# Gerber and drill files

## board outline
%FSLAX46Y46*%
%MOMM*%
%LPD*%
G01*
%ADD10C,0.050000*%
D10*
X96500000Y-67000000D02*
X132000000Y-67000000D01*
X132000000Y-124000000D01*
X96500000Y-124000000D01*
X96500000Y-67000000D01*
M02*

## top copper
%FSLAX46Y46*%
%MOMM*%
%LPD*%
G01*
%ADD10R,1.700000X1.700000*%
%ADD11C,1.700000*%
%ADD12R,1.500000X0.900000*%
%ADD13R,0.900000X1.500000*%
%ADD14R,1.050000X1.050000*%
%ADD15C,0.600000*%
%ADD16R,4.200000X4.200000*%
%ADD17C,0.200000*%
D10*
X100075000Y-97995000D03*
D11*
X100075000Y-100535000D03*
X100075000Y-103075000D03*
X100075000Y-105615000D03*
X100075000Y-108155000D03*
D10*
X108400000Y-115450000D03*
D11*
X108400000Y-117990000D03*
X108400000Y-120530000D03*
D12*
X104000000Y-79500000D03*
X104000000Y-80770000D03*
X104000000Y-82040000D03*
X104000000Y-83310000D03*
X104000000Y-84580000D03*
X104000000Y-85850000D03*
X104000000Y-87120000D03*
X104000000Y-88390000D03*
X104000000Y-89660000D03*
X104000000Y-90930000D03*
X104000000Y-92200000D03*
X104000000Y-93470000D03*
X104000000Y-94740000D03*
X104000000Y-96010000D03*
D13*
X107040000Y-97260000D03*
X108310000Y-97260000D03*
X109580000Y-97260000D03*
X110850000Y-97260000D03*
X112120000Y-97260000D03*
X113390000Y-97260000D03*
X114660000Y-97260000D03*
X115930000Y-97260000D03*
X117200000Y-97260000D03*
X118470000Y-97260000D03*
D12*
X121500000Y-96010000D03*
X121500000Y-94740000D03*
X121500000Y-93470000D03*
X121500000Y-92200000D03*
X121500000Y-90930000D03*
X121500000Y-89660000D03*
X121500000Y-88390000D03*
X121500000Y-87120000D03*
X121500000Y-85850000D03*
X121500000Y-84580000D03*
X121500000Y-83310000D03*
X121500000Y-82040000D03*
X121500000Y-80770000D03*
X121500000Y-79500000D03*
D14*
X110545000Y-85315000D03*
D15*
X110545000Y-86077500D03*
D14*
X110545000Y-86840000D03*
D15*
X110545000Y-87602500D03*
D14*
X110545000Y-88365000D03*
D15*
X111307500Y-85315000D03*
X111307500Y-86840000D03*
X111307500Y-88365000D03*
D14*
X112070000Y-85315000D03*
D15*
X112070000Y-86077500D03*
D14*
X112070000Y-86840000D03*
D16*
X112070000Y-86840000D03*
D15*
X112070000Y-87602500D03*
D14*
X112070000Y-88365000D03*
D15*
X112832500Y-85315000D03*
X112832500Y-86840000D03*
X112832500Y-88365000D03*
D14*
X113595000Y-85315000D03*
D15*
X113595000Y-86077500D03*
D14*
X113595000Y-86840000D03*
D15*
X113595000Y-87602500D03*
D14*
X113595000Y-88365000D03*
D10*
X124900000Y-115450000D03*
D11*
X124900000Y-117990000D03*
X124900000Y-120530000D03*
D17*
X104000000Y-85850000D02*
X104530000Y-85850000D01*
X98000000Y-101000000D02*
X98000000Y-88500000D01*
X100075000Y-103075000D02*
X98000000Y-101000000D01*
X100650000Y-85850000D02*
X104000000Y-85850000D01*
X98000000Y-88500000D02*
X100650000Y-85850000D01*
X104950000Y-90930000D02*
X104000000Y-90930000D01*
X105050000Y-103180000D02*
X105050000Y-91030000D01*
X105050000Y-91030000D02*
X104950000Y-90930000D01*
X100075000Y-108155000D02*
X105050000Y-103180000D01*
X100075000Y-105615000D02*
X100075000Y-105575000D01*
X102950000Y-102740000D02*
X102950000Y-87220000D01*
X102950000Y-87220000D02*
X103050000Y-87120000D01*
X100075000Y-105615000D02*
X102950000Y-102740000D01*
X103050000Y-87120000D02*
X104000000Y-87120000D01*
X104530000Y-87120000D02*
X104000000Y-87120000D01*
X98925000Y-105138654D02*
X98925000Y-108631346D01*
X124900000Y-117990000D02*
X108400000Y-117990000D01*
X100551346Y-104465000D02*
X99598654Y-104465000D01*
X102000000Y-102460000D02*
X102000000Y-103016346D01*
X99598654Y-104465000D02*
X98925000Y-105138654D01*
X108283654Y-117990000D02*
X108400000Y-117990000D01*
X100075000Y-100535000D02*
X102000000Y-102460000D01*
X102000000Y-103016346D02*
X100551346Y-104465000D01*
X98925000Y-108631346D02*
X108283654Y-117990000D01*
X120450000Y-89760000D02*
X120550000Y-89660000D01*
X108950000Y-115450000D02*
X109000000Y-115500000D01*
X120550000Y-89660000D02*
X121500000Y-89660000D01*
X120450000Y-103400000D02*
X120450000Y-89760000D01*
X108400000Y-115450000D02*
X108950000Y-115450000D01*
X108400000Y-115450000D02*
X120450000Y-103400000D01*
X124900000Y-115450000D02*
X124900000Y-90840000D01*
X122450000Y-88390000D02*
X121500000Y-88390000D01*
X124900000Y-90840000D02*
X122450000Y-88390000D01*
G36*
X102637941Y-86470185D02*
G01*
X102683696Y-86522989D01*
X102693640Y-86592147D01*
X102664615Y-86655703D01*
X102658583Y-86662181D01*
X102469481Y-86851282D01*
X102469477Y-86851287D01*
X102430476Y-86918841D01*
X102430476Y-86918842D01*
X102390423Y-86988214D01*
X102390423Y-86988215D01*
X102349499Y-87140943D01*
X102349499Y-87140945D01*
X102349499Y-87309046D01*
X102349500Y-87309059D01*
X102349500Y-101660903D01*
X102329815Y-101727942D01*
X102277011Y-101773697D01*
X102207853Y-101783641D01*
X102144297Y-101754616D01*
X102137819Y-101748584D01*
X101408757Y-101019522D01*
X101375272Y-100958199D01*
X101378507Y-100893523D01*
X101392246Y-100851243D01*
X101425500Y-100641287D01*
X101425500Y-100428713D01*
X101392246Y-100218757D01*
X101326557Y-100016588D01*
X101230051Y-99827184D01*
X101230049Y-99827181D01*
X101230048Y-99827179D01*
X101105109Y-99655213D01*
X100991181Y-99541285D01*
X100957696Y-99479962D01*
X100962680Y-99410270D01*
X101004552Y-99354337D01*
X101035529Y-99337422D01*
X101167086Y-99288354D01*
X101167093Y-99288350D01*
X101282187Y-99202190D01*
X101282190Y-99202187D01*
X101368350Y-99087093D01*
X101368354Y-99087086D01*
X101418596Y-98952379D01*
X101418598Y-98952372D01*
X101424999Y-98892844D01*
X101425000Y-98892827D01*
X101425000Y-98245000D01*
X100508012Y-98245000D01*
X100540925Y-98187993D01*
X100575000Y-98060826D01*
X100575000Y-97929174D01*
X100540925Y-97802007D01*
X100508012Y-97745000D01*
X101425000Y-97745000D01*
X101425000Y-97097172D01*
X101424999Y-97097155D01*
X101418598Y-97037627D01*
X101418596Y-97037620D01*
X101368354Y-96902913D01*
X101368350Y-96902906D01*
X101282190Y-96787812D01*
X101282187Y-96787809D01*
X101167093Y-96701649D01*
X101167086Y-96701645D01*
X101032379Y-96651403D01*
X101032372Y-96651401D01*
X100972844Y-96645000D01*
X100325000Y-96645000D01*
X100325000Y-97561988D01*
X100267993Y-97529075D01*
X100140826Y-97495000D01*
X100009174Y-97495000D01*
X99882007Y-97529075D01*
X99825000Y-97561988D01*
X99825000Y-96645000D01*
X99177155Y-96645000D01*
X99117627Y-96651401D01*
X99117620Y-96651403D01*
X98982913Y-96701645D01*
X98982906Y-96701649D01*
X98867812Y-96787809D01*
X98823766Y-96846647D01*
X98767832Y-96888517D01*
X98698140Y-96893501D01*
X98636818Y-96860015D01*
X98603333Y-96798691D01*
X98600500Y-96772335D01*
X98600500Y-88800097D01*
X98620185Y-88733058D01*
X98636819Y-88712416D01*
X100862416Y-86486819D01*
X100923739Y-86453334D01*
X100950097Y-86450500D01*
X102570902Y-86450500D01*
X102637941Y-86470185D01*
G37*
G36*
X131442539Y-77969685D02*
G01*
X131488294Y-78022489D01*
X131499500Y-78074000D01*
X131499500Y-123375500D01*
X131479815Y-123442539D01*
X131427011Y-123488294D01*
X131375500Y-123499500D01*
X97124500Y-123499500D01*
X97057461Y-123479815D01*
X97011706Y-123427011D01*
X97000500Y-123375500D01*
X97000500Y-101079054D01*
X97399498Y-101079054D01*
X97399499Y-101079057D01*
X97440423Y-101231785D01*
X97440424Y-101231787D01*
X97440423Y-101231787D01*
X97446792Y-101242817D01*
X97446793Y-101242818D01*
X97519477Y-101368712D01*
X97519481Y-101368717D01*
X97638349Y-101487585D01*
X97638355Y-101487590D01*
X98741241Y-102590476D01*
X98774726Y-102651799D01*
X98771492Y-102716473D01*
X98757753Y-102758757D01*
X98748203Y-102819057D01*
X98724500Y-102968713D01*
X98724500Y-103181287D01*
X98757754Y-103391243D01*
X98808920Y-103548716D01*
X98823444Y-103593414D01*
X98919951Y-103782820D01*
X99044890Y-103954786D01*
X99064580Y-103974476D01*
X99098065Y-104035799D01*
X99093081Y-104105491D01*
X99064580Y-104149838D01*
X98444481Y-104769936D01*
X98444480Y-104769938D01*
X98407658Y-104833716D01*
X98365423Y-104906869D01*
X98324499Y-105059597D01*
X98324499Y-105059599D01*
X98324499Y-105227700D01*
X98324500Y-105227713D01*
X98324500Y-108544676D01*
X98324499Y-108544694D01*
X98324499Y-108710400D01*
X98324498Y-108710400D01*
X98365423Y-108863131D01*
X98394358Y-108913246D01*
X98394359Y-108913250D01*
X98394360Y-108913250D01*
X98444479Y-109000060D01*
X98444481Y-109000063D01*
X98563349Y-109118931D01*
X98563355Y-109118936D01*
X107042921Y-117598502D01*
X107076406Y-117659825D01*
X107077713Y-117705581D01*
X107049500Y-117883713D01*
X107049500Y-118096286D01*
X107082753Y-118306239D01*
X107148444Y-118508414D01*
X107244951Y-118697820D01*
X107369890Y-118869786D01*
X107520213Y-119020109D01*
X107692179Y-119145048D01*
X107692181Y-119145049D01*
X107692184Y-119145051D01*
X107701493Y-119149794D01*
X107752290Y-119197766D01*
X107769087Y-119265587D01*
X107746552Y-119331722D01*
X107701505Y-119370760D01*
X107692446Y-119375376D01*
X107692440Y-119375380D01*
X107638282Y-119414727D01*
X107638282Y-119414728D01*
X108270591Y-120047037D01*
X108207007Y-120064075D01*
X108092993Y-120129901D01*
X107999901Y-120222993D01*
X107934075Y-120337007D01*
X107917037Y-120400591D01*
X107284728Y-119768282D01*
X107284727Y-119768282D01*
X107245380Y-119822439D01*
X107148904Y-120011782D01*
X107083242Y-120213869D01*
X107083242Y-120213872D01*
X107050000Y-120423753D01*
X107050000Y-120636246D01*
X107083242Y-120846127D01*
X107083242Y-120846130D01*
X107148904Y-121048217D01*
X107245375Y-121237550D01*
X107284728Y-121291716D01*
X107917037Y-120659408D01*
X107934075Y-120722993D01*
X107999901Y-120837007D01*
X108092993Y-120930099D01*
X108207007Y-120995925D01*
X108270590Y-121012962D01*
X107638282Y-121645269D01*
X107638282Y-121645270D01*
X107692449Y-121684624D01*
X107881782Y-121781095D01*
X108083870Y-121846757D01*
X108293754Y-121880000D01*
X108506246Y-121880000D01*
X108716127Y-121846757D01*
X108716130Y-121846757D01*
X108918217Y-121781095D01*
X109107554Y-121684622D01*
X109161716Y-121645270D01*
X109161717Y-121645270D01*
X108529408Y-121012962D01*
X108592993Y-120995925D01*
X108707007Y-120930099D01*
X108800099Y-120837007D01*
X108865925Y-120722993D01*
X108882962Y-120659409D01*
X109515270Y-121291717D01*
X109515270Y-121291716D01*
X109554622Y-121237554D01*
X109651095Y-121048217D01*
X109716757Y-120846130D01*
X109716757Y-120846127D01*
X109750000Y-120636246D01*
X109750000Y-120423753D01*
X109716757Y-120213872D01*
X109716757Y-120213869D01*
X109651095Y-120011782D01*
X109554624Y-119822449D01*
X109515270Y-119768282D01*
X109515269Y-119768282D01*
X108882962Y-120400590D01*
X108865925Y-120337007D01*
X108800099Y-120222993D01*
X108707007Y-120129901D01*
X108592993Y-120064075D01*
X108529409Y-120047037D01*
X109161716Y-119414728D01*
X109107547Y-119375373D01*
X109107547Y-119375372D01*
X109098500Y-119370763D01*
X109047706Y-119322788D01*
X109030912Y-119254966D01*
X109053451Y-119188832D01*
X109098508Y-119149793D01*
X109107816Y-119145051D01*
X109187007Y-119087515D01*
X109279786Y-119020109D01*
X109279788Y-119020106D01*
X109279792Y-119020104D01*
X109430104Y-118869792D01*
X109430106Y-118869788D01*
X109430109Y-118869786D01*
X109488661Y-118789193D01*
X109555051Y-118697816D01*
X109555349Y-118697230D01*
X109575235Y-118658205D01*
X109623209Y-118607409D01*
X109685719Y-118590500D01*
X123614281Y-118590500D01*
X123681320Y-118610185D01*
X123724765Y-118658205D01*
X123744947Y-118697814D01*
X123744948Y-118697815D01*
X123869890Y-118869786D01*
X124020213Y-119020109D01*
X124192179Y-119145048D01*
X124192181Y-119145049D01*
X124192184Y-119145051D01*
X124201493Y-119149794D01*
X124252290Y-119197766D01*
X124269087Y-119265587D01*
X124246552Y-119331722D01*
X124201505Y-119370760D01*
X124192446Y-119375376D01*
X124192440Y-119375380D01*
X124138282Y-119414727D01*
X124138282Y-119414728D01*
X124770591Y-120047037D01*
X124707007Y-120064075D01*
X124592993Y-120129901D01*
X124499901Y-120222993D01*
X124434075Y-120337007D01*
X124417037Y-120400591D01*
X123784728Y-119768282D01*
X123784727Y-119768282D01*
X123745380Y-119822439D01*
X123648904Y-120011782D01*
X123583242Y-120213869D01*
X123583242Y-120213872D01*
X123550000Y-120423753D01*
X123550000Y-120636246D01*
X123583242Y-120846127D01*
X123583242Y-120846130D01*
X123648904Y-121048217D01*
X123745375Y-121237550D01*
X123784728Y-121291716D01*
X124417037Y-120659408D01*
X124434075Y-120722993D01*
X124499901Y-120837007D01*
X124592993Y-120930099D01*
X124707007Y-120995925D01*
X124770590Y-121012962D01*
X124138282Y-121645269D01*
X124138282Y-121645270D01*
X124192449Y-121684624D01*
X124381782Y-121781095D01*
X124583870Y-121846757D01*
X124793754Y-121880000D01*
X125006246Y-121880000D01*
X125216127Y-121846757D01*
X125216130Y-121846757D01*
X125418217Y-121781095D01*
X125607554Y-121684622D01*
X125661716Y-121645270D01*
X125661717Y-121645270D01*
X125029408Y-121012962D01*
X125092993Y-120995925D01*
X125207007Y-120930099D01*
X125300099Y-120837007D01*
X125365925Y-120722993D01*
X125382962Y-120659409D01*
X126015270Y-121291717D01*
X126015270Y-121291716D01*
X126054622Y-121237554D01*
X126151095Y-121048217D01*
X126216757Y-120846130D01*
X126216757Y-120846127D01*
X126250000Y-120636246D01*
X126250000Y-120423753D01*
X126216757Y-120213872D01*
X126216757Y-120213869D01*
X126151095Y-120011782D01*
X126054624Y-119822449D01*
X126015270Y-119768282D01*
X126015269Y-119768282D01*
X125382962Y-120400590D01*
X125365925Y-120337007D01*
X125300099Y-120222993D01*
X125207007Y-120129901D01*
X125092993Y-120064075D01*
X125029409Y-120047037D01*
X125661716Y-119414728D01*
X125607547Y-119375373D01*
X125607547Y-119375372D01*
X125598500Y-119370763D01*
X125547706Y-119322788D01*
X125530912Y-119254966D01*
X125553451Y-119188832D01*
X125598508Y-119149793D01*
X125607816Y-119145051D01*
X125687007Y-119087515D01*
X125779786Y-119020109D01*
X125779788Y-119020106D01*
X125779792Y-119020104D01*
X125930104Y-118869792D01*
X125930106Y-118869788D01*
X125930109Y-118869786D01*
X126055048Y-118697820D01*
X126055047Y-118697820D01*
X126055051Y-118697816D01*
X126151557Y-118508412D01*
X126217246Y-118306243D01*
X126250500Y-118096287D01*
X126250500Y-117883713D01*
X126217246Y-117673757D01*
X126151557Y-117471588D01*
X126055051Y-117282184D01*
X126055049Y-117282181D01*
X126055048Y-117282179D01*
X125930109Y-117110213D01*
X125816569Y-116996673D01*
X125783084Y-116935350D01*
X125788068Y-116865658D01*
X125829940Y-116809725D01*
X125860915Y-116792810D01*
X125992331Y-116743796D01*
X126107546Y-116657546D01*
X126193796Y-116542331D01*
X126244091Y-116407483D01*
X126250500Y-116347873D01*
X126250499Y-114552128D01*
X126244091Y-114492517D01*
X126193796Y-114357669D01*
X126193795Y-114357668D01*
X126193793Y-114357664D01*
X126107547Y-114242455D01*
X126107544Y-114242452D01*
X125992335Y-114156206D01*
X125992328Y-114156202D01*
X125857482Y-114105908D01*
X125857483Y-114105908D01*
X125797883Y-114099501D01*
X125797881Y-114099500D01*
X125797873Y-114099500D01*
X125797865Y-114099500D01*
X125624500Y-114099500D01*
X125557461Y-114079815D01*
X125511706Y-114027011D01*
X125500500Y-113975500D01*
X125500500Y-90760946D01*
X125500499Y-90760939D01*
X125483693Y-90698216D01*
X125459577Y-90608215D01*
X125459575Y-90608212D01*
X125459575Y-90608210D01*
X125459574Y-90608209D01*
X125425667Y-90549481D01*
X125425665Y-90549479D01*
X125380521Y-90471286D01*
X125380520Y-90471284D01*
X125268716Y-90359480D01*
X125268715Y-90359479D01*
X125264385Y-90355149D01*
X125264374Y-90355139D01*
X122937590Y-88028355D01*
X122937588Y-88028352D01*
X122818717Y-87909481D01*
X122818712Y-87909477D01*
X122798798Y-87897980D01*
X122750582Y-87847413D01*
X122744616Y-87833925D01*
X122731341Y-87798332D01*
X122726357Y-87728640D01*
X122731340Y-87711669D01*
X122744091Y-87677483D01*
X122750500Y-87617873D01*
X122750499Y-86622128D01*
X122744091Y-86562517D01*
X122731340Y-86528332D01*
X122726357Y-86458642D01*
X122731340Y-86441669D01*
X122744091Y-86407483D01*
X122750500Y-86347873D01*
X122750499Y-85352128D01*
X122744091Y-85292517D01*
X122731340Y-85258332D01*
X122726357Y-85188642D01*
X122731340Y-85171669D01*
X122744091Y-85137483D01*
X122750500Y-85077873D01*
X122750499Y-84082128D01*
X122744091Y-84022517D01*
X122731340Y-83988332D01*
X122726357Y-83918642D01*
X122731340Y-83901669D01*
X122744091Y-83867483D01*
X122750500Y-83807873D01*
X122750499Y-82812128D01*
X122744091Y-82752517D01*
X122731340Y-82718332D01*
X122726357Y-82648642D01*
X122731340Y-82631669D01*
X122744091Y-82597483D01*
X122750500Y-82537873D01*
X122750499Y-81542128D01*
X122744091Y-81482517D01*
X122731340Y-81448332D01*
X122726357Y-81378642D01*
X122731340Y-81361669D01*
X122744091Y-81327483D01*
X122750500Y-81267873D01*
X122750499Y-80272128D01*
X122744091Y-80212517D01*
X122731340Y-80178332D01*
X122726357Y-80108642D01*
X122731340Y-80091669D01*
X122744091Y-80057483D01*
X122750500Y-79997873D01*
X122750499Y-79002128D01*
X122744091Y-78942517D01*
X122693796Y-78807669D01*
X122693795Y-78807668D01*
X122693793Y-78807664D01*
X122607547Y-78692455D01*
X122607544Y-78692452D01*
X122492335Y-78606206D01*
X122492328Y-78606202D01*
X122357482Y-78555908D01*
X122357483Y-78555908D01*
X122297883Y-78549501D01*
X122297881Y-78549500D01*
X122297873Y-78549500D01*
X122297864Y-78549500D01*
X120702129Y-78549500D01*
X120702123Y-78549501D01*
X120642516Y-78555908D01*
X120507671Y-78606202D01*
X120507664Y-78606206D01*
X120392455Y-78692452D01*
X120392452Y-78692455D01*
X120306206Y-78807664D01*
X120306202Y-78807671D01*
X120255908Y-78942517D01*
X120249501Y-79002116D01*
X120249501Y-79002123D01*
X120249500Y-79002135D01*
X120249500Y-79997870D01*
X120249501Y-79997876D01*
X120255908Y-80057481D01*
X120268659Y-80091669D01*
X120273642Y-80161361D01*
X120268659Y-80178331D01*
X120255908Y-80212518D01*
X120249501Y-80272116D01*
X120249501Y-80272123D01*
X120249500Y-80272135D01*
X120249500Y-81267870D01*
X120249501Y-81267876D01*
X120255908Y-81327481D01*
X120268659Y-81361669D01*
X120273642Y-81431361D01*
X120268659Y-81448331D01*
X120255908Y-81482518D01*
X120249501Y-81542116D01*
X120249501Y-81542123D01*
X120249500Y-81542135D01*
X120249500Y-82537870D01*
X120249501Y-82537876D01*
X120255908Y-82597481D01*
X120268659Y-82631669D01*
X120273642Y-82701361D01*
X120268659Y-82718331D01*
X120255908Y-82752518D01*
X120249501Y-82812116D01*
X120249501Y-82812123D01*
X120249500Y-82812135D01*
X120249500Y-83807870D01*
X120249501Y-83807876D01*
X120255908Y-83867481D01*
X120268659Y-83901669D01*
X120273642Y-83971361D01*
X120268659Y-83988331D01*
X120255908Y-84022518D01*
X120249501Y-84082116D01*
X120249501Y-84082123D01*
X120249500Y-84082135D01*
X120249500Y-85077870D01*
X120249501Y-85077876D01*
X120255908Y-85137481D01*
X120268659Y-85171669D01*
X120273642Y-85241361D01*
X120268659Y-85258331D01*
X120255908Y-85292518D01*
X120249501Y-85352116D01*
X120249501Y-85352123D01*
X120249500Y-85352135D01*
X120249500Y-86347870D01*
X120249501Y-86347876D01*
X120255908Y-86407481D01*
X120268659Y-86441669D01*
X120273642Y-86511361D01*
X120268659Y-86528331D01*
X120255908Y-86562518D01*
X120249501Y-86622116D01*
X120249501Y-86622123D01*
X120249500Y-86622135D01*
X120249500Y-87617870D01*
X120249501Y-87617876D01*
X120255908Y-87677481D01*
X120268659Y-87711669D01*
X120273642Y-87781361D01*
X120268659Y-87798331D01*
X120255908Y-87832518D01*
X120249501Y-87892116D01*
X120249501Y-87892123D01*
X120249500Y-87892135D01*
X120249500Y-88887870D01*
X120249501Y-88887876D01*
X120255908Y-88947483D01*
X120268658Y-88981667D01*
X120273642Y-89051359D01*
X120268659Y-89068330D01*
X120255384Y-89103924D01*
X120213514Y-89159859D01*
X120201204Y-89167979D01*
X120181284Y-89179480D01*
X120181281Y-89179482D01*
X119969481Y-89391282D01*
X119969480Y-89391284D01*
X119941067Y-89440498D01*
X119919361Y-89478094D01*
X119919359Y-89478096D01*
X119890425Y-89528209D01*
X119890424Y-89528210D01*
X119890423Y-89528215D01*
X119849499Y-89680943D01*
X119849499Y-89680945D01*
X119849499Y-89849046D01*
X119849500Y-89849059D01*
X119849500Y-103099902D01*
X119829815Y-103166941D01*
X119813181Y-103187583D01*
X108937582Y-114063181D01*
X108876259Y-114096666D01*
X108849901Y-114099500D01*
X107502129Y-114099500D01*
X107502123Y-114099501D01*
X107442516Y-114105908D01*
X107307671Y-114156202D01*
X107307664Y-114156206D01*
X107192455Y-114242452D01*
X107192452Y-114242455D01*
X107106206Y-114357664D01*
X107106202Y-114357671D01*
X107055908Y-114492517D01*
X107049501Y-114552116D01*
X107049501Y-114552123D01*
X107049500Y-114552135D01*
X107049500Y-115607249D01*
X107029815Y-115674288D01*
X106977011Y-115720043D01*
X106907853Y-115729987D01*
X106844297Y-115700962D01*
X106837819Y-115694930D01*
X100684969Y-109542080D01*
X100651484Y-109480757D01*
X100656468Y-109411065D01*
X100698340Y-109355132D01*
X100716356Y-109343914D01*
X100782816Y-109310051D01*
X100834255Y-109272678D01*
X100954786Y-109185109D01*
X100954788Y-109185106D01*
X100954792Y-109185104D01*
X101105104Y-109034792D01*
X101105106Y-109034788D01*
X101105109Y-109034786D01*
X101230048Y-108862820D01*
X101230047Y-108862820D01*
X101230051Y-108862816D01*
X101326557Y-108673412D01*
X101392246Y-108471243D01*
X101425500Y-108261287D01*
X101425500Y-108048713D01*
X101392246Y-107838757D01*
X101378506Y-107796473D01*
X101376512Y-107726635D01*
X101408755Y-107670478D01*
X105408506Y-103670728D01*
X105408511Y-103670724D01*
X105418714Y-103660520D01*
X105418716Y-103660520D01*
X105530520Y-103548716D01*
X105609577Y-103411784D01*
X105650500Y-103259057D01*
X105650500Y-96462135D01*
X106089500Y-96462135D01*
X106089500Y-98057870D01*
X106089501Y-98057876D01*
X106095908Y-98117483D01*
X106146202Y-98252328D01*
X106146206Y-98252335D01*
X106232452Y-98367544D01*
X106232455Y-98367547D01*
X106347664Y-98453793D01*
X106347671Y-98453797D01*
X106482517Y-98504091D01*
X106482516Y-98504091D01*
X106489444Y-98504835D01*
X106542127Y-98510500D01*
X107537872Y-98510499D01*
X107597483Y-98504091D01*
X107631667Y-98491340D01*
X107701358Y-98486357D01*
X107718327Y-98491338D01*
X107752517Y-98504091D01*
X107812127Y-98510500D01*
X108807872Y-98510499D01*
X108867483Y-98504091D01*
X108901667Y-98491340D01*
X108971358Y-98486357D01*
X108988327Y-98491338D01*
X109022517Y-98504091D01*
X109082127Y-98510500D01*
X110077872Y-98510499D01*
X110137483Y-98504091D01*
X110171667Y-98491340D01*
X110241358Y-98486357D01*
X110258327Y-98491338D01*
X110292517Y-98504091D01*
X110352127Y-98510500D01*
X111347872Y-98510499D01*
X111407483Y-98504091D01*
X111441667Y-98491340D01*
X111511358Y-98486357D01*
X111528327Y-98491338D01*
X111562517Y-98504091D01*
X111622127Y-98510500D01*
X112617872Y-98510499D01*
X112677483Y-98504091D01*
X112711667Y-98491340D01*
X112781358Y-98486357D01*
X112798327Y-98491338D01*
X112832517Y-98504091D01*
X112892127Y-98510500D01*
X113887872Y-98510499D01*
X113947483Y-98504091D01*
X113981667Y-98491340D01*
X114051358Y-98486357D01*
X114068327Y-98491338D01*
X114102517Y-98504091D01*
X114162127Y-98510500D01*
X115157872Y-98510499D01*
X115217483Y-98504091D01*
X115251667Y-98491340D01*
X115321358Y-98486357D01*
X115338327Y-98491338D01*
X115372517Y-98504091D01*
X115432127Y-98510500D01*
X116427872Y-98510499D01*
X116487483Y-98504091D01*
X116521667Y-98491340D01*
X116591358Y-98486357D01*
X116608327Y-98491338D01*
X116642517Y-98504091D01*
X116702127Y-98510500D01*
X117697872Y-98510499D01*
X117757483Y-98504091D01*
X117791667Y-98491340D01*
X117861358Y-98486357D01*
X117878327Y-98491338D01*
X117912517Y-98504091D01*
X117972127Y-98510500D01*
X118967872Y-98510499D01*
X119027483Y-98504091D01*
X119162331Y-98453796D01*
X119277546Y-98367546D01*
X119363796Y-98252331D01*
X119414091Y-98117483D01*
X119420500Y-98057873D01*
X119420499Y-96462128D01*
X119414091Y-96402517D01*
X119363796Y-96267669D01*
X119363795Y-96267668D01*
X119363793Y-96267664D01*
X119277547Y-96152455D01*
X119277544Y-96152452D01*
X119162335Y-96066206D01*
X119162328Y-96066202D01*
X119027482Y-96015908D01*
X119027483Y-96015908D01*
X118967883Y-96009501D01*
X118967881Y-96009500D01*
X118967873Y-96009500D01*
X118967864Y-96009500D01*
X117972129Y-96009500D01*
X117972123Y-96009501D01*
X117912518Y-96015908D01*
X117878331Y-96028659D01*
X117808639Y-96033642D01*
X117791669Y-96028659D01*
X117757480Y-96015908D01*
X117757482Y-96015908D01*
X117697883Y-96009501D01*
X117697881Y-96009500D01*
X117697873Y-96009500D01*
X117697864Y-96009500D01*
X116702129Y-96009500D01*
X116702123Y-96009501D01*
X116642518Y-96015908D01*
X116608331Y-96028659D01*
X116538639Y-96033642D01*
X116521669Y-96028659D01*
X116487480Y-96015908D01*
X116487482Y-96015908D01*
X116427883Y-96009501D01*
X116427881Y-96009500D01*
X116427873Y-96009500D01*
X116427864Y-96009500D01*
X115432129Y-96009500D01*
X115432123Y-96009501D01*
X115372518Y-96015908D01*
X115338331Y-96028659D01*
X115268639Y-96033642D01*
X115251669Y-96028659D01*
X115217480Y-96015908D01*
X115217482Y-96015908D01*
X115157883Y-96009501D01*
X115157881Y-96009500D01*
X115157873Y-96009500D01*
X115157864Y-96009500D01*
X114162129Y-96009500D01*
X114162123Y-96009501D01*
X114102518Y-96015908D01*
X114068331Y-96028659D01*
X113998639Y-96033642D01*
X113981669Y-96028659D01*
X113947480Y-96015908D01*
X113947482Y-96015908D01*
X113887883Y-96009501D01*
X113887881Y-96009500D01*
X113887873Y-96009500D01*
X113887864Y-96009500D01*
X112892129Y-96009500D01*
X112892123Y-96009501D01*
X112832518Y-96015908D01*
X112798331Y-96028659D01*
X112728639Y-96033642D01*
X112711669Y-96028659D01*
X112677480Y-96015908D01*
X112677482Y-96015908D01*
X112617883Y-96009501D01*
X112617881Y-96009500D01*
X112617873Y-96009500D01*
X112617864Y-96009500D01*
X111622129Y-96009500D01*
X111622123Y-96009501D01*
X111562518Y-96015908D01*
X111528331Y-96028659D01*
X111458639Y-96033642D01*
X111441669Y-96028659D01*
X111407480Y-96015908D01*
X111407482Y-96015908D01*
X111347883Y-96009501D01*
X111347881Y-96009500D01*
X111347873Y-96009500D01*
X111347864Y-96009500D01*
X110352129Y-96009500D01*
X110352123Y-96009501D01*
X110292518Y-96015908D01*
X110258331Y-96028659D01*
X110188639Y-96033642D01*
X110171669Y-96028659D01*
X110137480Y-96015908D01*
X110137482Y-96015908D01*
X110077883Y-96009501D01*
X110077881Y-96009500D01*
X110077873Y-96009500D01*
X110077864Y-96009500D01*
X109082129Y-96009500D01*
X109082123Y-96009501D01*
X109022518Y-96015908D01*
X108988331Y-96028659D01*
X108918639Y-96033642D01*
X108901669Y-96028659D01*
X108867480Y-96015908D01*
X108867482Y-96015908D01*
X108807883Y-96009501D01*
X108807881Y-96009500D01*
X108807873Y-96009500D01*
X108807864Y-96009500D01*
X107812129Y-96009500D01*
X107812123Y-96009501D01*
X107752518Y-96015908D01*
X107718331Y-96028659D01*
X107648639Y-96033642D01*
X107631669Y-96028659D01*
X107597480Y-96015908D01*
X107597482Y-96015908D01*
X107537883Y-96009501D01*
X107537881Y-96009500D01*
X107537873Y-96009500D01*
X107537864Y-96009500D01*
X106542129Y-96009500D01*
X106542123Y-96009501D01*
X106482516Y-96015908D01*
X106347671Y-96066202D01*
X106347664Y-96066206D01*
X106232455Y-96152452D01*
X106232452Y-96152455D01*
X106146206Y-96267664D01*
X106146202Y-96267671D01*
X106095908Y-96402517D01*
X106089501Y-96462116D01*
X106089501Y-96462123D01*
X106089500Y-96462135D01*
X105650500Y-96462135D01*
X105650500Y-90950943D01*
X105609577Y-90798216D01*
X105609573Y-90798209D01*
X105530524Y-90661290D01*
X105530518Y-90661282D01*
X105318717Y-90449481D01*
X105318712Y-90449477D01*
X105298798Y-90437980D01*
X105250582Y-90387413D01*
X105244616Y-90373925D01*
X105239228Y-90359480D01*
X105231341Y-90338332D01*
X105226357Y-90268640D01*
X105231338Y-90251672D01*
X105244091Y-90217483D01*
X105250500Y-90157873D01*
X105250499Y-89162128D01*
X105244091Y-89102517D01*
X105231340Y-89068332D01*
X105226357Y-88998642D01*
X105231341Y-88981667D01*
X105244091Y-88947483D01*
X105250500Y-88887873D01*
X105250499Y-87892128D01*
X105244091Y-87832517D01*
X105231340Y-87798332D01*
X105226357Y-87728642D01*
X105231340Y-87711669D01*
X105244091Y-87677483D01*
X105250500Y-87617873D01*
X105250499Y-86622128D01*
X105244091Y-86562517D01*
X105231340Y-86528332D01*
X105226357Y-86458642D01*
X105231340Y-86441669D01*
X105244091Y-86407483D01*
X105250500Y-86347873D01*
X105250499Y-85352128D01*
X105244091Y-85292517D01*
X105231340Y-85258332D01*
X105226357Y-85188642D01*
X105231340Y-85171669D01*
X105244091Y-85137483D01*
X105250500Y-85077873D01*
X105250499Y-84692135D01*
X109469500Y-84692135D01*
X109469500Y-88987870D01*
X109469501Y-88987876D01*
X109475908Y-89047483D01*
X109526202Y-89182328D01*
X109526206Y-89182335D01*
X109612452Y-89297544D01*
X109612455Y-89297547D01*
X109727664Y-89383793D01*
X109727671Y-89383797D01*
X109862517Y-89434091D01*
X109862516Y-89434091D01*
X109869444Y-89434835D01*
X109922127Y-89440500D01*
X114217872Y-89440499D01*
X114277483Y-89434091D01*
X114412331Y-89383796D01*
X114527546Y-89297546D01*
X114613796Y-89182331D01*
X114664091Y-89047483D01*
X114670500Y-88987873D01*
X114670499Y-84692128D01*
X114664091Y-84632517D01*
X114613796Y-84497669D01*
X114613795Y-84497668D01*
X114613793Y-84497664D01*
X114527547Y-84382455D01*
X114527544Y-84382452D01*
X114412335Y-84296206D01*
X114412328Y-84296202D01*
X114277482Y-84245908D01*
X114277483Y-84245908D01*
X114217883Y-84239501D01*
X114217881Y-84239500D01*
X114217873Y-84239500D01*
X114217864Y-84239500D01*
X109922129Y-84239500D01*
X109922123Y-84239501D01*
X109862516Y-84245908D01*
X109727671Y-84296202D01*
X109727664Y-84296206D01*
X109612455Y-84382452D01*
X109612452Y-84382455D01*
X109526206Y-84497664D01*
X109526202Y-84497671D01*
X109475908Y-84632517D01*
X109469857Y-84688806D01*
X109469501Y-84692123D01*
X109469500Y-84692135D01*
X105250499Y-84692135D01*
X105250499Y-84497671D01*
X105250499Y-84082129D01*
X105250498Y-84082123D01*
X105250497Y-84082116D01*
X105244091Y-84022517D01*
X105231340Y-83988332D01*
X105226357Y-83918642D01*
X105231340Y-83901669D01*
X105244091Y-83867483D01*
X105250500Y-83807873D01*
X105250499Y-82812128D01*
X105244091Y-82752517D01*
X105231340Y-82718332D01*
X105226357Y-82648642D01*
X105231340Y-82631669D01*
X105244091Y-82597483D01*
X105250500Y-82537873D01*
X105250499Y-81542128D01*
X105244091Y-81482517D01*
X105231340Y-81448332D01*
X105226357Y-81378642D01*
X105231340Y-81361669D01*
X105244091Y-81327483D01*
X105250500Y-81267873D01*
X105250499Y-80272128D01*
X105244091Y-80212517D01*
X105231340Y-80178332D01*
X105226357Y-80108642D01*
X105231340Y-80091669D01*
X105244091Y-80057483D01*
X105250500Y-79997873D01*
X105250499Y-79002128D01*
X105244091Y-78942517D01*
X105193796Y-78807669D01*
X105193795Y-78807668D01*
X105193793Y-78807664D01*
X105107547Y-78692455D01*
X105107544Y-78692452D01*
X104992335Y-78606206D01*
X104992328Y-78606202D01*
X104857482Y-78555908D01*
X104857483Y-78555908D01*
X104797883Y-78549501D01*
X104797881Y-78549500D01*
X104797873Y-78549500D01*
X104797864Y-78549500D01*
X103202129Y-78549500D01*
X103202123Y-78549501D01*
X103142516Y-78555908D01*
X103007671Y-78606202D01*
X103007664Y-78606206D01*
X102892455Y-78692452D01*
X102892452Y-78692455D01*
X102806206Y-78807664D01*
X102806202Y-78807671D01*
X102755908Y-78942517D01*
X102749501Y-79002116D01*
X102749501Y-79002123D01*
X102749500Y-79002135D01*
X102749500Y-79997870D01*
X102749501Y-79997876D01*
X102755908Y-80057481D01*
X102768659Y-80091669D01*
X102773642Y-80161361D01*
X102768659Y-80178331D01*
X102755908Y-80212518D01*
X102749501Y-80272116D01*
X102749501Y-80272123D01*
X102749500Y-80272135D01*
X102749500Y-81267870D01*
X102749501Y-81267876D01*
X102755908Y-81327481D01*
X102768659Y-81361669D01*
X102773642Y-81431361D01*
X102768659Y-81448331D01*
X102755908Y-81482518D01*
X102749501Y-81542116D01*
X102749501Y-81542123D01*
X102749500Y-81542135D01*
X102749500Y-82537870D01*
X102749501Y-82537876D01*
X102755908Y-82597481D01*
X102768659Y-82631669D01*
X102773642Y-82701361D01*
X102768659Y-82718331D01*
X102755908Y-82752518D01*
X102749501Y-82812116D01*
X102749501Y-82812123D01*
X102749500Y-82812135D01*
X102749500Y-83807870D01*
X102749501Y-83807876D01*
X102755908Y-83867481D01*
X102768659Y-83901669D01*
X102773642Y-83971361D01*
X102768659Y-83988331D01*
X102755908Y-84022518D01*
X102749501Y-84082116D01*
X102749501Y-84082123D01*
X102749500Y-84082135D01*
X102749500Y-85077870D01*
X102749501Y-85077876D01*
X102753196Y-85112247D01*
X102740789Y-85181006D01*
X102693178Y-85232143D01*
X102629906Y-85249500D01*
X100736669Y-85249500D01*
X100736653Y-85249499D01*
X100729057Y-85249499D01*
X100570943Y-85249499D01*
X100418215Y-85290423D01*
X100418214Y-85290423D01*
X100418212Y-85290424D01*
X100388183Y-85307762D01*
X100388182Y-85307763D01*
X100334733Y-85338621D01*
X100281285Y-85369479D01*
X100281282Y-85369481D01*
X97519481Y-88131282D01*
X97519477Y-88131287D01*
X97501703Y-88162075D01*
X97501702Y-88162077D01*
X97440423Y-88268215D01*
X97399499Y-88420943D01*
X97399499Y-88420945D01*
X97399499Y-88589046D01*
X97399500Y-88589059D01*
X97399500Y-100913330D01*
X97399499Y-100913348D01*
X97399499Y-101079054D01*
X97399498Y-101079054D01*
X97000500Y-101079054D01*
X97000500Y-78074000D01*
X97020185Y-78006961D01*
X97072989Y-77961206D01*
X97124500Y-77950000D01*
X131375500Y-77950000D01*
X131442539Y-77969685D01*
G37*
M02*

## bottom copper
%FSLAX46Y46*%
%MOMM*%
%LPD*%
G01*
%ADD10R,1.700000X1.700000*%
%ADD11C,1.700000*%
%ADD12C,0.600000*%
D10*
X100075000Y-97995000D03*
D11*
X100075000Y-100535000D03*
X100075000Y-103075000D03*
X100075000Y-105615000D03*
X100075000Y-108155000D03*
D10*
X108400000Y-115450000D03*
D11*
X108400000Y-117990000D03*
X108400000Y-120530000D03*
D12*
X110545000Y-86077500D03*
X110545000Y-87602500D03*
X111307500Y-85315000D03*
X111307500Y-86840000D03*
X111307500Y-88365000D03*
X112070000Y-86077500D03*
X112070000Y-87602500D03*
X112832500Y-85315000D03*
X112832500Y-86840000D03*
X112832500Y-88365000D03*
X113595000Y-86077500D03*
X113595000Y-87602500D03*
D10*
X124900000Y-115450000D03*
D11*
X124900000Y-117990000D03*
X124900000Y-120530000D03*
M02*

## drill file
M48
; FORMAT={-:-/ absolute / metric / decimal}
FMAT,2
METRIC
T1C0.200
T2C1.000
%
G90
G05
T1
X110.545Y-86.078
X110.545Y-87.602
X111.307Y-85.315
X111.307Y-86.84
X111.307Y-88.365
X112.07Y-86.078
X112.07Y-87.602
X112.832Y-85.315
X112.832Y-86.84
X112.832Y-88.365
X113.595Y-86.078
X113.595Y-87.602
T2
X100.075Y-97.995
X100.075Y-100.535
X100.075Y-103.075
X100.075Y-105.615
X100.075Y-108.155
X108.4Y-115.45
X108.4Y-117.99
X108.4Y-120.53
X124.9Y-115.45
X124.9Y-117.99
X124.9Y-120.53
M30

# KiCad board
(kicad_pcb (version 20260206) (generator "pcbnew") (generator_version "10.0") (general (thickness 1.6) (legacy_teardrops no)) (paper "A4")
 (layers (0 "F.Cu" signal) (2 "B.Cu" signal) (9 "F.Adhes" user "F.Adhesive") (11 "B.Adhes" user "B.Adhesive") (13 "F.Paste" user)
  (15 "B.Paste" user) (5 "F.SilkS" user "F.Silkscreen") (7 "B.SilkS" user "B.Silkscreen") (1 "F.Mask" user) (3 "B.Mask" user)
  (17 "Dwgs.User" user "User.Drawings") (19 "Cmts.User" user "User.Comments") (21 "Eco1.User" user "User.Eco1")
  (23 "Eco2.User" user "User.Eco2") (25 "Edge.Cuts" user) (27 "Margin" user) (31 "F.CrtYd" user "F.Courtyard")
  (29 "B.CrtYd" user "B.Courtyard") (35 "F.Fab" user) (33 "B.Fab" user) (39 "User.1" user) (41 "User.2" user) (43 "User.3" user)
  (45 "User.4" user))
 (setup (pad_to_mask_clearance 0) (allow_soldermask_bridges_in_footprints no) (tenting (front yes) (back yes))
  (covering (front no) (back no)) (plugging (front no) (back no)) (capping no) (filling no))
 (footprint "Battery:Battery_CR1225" (layer "F.Cu") (at 113 107)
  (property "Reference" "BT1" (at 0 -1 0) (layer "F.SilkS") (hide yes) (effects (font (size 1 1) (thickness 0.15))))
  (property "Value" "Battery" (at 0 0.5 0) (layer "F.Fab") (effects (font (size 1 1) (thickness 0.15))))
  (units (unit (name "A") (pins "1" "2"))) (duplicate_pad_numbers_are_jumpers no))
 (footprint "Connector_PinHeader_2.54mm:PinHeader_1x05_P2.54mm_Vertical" (layer "F.Cu") (at 100.075 97.995)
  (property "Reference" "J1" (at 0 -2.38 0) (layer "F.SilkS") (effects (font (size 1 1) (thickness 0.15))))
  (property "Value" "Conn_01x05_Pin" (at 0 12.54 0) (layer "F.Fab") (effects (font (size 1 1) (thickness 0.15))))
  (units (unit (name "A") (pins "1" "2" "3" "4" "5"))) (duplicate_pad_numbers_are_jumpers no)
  (pad "1" thru_hole rect (at 0 0) (size 1.7 1.7) (drill 1) (layers "*.Cu" "*.Mask") (remove_unused_layers no) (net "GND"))
  (pad "2" thru_hole circle (at 0 2.54) (size 1.7 1.7) (drill 1) (layers "*.Cu" "*.Mask") (remove_unused_layers no) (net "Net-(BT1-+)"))
  (pad "3" thru_hole circle (at 0 5.08) (size 1.7 1.7) (drill 1) (layers "*.Cu" "*.Mask") (remove_unused_layers no) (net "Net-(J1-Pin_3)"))
  (pad "4" thru_hole circle (at 0 7.62) (size 1.7 1.7) (drill 1) (layers "*.Cu" "*.Mask") (remove_unused_layers no) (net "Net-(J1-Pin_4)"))
  (pad "5" thru_hole circle (at 0 10.16) (size 1.7 1.7) (drill 1) (layers "*.Cu" "*.Mask") (remove_unused_layers no) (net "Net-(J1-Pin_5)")))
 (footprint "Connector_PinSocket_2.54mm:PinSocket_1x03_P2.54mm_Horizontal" (layer "F.Cu") (at 108.4 115.45)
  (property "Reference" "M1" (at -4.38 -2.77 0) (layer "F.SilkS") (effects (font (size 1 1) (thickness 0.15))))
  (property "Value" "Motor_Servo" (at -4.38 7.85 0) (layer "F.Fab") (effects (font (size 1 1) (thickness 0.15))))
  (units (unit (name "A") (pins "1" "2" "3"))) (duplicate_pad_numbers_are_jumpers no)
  (pad "1" thru_hole rect (at 0 0) (size 1.7 1.7) (drill 1) (layers "*.Cu" "*.Mask") (remove_unused_layers no) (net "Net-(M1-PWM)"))
  (pad "2" thru_hole circle (at 0 2.54) (size 1.7 1.7) (drill 1) (layers "*.Cu" "*.Mask") (remove_unused_layers no) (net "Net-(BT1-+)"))
  (pad "3" thru_hole circle (at 0 5.08) (size 1.7 1.7) (drill 1) (layers "*.Cu" "*.Mask") (remove_unused_layers no) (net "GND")))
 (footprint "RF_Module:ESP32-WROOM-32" (layer "F.Cu") (at 112.75 87.75)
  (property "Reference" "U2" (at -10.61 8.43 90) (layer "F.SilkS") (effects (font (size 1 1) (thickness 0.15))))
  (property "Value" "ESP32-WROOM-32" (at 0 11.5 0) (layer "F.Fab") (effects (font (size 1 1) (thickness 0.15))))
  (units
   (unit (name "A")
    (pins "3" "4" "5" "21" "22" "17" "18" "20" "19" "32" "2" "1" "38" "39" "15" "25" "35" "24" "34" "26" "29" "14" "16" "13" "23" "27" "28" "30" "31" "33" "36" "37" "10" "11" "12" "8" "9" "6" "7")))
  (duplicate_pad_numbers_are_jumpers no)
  (pad "1" smd rect (at -8.75 -8.25) (size 1.5 0.9) (layers "F.Cu" "F.Mask" "F.Paste") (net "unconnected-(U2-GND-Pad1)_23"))
  (pad "2" smd rect (at -8.75 -6.98) (size 1.5 0.9) (layers "F.Cu" "F.Mask" "F.Paste") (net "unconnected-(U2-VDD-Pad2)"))
  (pad "3" smd rect (at -8.75 -5.71) (size 1.5 0.9) (layers "F.Cu" "F.Mask" "F.Paste") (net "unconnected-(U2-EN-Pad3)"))
  (pad "4" smd rect (at -8.75 -4.44) (size 1.5 0.9) (layers "F.Cu" "F.Mask" "F.Paste") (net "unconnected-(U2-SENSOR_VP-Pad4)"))
  (pad "5" smd rect (at -8.75 -3.17) (size 1.5 0.9) (layers "F.Cu" "F.Mask" "F.Paste") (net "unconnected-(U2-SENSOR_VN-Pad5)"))
  (pad "6" smd rect (at -8.75 -1.9) (size 1.5 0.9) (layers "F.Cu" "F.Mask" "F.Paste") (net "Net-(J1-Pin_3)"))
  (pad "7" smd rect (at -8.75 -0.63) (size 1.5 0.9) (layers "F.Cu" "F.Mask" "F.Paste") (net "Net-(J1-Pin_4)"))
  (pad "8" smd rect (at -8.75 0.64) (size 1.5 0.9) (layers "F.Cu" "F.Mask" "F.Paste") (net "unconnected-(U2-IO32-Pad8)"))
  (pad "9" smd rect (at -8.75 1.91) (size 1.5 0.9) (layers "F.Cu" "F.Mask" "F.Paste") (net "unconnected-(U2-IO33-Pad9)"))
  (pad "10" smd rect (at -8.75 3.18) (size 1.5 0.9) (layers "F.Cu" "F.Mask" "F.Paste") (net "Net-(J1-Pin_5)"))
  (pad "11" smd rect (at -8.75 4.45) (size 1.5 0.9) (layers "F.Cu" "F.Mask" "F.Paste") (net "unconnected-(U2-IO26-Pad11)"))
  (pad "12" smd rect (at -8.75 5.72) (size 1.5 0.9) (layers "F.Cu" "F.Mask" "F.Paste") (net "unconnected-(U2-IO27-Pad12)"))
  (pad "13" smd rect (at -8.75 6.99) (size 1.5 0.9) (layers "F.Cu" "F.Mask" "F.Paste") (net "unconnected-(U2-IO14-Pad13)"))
  (pad "14" smd rect (at -8.75 8.26) (size 1.5 0.9) (layers "F.Cu" "F.Mask" "F.Paste") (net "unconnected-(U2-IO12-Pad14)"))
  (pad "15" smd rect (at -5.71 9.51 90) (size 1.5 0.9) (layers "F.Cu" "F.Mask" "F.Paste") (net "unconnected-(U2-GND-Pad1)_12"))
  (pad "16" smd rect (at -4.44 9.51 90) (size 1.5 0.9) (layers "F.Cu" "F.Mask" "F.Paste") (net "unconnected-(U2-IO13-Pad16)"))
  (pad "17" smd rect (at -3.17 9.51 90) (size 1.5 0.9) (layers "F.Cu" "F.Mask" "F.Paste") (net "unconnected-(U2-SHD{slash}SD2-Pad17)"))
  (pad "18" smd rect (at -1.9 9.51 90) (size 1.5 0.9) (layers "F.Cu" "F.Mask" "F.Paste") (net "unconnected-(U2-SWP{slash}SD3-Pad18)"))
  (pad "19" smd rect (at -0.63 9.51 90) (size 1.5 0.9) (layers "F.Cu" "F.Mask" "F.Paste") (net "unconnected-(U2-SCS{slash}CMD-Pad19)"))
  (pad "20" smd rect (at 0.64 9.51 90) (size 1.5 0.9) (layers "F.Cu" "F.Mask" "F.Paste") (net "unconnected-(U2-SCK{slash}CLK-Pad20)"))
  (pad "21" smd rect (at 1.91 9.51 90) (size 1.5 0.9) (layers "F.Cu" "F.Mask" "F.Paste") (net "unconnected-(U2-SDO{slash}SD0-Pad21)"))
  (pad "22" smd rect (at 3.18 9.51 90) (size 1.5 0.9) (layers "F.Cu" "F.Mask" "F.Paste") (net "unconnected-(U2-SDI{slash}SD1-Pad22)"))
  (pad "23" smd rect (at 4.45 9.51 90) (size 1.5 0.9) (layers "F.Cu" "F.Mask" "F.Paste") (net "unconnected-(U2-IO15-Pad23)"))
  (pad "24" smd rect (at 5.72 9.51 90) (size 1.5 0.9) (layers "F.Cu" "F.Mask" "F.Paste") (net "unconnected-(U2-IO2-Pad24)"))
  (pad "25" smd rect (at 8.75 8.26) (size 1.5 0.9) (layers "F.Cu" "F.Mask" "F.Paste") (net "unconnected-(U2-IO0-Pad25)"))
  (pad "26" smd rect (at 8.75 6.99) (size 1.5 0.9) (layers "F.Cu" "F.Mask" "F.Paste") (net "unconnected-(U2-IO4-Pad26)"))
  (pad "27" smd rect (at 8.75 5.72) (size 1.5 0.9) (layers "F.Cu" "F.Mask" "F.Paste") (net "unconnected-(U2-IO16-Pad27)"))
  (pad "28" smd rect (at 8.75 4.45) (size 1.5 0.9) (layers "F.Cu" "F.Mask" "F.Paste") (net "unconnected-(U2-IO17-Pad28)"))
  (pad "29" smd rect (at 8.75 3.18) (size 1.5 0.9) (layers "F.Cu" "F.Mask" "F.Paste") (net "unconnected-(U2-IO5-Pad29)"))
  (pad "30" smd rect (at 8.75 1.91) (size 1.5 0.9) (layers "F.Cu" "F.Mask" "F.Paste") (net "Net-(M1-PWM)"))
  (pad "31" smd rect (at 8.75 0.64) (size 1.5 0.9) (layers "F.Cu" "F.Mask" "F.Paste") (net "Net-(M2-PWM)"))
  (pad "32" smd rect (at 8.75 -0.63) (size 1.5 0.9) (layers "F.Cu" "F.Mask" "F.Paste") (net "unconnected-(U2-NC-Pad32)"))
  (pad "33" smd rect (at 8.75 -1.9) (size 1.5 0.9) (layers "F.Cu" "F.Mask" "F.Paste") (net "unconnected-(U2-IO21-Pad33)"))
  (pad "34" smd rect (at 8.75 -3.17) (size 1.5 0.9) (layers "F.Cu" "F.Mask" "F.Paste") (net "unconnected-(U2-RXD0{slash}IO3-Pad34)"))
  (pad "35" smd rect (at 8.75 -4.44) (size 1.5 0.9) (layers "F.Cu" "F.Mask" "F.Paste") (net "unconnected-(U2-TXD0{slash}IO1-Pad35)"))
  (pad "36" smd rect (at 8.75 -5.71) (size 1.5 0.9) (layers "F.Cu" "F.Mask" "F.Paste") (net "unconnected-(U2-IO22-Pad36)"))
  (pad "37" smd rect (at 8.75 -6.98) (size 1.5 0.9) (layers "F.Cu" "F.Mask" "F.Paste") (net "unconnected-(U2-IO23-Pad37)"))
  (pad "38" smd rect (at 8.75 -8.25) (size 1.5 0.9) (layers "F.Cu" "F.Mask" "F.Paste") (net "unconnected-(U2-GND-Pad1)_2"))
  (pad "39" smd rect (at -2.205 -2.435) (size 1.05 1.05) (layers "F.Cu" "F.Paste") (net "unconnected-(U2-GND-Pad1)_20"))
  (pad "39" thru_hole circle (at -2.205 -1.6725) (size 0.6 0.6) (drill 0.2) (layers "*.Cu" "F.Mask") (remove_unused_layers no)
   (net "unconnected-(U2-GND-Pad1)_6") (zone_connect 2))
  (pad "39" smd rect (at -2.205 -0.91) (size 1.05 1.05) (layers "F.Cu" "F.Paste") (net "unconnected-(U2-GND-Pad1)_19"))
  (pad "39" thru_hole circle (at -2.205 -0.1475) (size 0.6 0.6) (drill 0.2) (layers "*.Cu" "F.Mask") (remove_unused_layers no)
   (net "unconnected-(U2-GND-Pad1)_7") (zone_connect 2))
  (pad "39" smd rect (at -2.205 0.615) (size 1.05 1.05) (layers "F.Cu" "F.Paste") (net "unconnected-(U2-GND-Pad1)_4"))
  (pad "39" thru_hole circle (at -1.4425 -2.435) (size 0.6 0.6) (drill 0.2) (layers "*.Cu" "F.Mask") (remove_unused_layers no)
   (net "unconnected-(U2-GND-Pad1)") (zone_connect 2))
  (pad "39" thru_hole circle (at -1.4425 -0.91) (size 0.6 0.6) (drill 0.2) (layers "*.Cu" "F.Mask") (remove_unused_layers no)
   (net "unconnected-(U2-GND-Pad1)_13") (zone_connect 2))
  (pad "39" thru_hole circle (at -1.4425 0.615) (size 0.6 0.6) (drill 0.2) (layers "*.Cu" "F.Mask") (remove_unused_layers no)
   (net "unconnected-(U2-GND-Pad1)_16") (zone_connect 2))
  (pad "39" smd rect (at -0.68 -2.435) (size 1.05 1.05) (layers "F.Cu" "F.Paste") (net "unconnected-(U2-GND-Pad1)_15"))
  (pad "39" thru_hole circle (at -0.68 -1.6725) (size 0.6 0.6) (drill 0.2) (layers "*.Cu" "F.Mask") (remove_unused_layers no)
   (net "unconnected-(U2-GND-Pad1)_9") (zone_connect 2))
  (pad "39" smd rect (at -0.68 -0.91) (size 1.05 1.05) (layers "F.Cu" "F.Paste") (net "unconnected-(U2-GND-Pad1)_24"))
  (pad "39" smd rect (at -0.68 -0.91) (size 4.2 4.2) (layers "F.Cu" "F.Mask") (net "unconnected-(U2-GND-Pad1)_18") (zone_connect 2))
  (pad "39" thru_hole circle (at -0.68 -0.1475) (size 0.6 0.6) (drill 0.2) (layers "*.Cu" "F.Mask") (remove_unused_layers no)
   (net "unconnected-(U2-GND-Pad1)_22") (zone_connect 2))
  (pad "39" smd rect (at -0.68 0.615) (size 1.05 1.05) (layers "F.Cu" "F.Paste") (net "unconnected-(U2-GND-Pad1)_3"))
  (pad "39" thru_hole circle (at 0.0825 -2.435) (size 0.6 0.6) (drill 0.2) (layers "*.Cu" "F.Mask") (remove_unused_layers no)
   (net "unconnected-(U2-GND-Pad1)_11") (zone_connect 2))
  (pad "39" thru_hole circle (at 0.0825 -0.91) (size 0.6 0.6) (drill 0.2) (layers "*.Cu" "F.Mask") (remove_unused_layers no)
   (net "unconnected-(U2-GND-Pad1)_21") (zone_connect 2))
  (pad "39" thru_hole circle (at 0.0825 0.615) (size 0.6 0.6) (drill 0.2) (layers "*.Cu" "F.Mask") (remove_unused_layers no)
   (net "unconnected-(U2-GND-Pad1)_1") (zone_connect 2))
  (pad "39" smd rect (at 0.845 -2.435) (size 1.05 1.05) (layers "F.Cu" "F.Paste") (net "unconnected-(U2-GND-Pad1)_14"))
  (pad "39" thru_hole circle (at 0.845 -1.6725) (size 0.6 0.6) (drill 0.2) (layers "*.Cu" "F.Mask") (remove_unused_layers no)
   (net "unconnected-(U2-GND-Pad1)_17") (zone_connect 2))
  (pad "39" smd rect (at 0.845 -0.91) (size 1.05 1.05) (layers "F.Cu" "F.Paste") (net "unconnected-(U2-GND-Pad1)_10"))
  (pad "39" thru_hole circle (at 0.845 -0.1475) (size 0.6 0.6) (drill 0.2) (layers "*.Cu" "F.Mask") (remove_unused_layers no)
   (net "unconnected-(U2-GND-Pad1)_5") (zone_connect 2))
  (pad "39" smd rect (at 0.845 0.615) (size 1.05 1.05) (layers "F.Cu" "F.Paste") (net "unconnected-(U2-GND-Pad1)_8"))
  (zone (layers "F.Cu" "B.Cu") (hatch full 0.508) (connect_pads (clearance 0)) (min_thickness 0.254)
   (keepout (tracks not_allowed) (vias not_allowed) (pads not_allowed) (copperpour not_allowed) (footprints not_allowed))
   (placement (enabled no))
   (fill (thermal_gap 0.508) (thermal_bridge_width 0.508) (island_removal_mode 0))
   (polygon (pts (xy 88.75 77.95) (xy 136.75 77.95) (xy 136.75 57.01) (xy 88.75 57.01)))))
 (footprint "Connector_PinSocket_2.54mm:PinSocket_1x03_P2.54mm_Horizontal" (layer "F.Cu") (at 124.9 115.45)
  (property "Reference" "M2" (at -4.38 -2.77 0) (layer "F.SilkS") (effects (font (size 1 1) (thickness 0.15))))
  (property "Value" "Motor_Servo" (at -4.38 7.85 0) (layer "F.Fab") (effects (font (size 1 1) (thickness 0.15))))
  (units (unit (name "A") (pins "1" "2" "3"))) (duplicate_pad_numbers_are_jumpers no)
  (pad "1" thru_hole rect (at 0 0) (size 1.7 1.7) (drill 1) (layers "*.Cu" "*.Mask") (remove_unused_layers no) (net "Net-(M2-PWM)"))
  (pad "2" thru_hole circle (at 0 2.54) (size 1.7 1.7) (drill 1) (layers "*.Cu" "*.Mask") (remove_unused_layers no) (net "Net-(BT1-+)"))
  (pad "3" thru_hole circle (at 0 5.08) (size 1.7 1.7) (drill 1) (layers "*.Cu" "*.Mask") (remove_unused_layers no) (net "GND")))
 (gr_rect (start 96.5 67) (end 132 124) (stroke (width 0.05) (type default)) (fill no) (layer "Edge.Cuts"))
 (segment (start 104 85.85) (end 104.53 85.85) (width 0.2) (layer "F.Cu") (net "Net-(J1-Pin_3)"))
 (segment (start 98 101) (end 98 88.5) (width 0.2) (layer "F.Cu") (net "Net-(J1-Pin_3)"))
 (segment (start 100.075 103.075) (end 98 101) (width 0.2) (layer "F.Cu") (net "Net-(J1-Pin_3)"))
 (segment (start 100.65 85.85) (end 104 85.85) (width 0.2) (layer "F.Cu") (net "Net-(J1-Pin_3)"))
 (segment (start 98 88.5) (end 100.65 85.85) (width 0.2) (layer "F.Cu") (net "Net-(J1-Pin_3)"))
 (segment (start 104.95 90.93) (end 104 90.93) (width 0.2) (layer "F.Cu") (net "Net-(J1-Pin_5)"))
 (segment (start 105.05 103.18) (end 105.05 91.03) (width 0.2) (layer "F.Cu") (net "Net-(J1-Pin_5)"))
 (segment (start 105.05 91.03) (end 104.95 90.93) (width 0.2) (layer "F.Cu") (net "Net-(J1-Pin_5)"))
 (segment (start 100.075 108.155) (end 105.05 103.18) (width 0.2) (layer "F.Cu") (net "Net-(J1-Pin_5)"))
 (segment (start 100.075 105.615) (end 100.075 105.575) (width 0.2) (layer "F.Cu") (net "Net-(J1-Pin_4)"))
 (segment (start 102.95 102.74) (end 102.95 87.22) (width 0.2) (layer "F.Cu") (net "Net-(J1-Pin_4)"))
 (segment (start 102.95 87.22) (end 103.05 87.12) (width 0.2) (layer "F.Cu") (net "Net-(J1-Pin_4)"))
 (segment (start 100.075 105.615) (end 102.95 102.74) (width 0.2) (layer "F.Cu") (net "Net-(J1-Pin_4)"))
 (segment (start 103.05 87.12) (end 104 87.12) (width 0.2) (layer "F.Cu") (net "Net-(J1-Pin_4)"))
 (segment (start 104.53 87.12) (end 104 87.12) (width 0.2) (layer "F.Cu") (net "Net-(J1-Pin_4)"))
 (segment (start 98.925 105.138654) (end 98.925 108.631346) (width 0.2) (layer "F.Cu") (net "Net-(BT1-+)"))
 (segment (start 124.9 117.99) (end 108.4 117.99) (width 0.2) (layer "F.Cu") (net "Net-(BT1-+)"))
 (segment (start 100.551346 104.465) (end 99.598654 104.465) (width 0.2) (layer "F.Cu") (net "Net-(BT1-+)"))
 (segment (start 102 102.46) (end 102 103.016346) (width 0.2) (layer "F.Cu") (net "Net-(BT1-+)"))
 (segment (start 99.598654 104.465) (end 98.925 105.138654) (width 0.2) (layer "F.Cu") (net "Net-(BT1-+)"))
 (segment (start 108.283654 117.99) (end 108.4 117.99) (width 0.2) (layer "F.Cu") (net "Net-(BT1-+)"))
 (segment (start 100.075 100.535) (end 102 102.46) (width 0.2) (layer "F.Cu") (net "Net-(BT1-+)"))
 (segment (start 102 103.016346) (end 100.551346 104.465) (width 0.2) (layer "F.Cu") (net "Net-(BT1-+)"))
 (segment (start 98.925 108.631346) (end 108.283654 117.99) (width 0.2) (layer "F.Cu") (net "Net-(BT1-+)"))
 (segment (start 120.45 89.76) (end 120.55 89.66) (width 0.2) (layer "F.Cu") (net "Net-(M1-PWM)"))
 (segment (start 108.95 115.45) (end 109 115.5) (width 0.2) (layer "F.Cu") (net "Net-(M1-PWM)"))
 (segment (start 120.55 89.66) (end 121.5 89.66) (width 0.2) (layer "F.Cu") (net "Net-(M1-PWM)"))
 (segment (start 120.45 103.4) (end 120.45 89.76) (width 0.2) (layer "F.Cu") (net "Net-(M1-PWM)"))
 (segment (start 108.4 115.45) (end 108.95 115.45) (width 0.2) (layer "F.Cu") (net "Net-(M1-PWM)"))
 (segment (start 108.4 115.45) (end 120.45 103.4) (width 0.2) (layer "F.Cu") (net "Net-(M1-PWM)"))
 (segment (start 124.9 115.45) (end 124.9 90.84) (width 0.2) (layer "F.Cu") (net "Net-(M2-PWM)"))
 (segment (start 122.45 88.39) (end 121.5 88.39) (width 0.2) (layer "F.Cu") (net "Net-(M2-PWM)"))
 (segment (start 124.9 90.84) (end 122.45 88.39) (width 0.2) (layer "F.Cu") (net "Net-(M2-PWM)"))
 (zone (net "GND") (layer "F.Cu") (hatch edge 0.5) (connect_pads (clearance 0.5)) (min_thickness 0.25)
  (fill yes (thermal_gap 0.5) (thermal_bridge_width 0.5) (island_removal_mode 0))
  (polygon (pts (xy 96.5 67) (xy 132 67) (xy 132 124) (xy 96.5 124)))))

